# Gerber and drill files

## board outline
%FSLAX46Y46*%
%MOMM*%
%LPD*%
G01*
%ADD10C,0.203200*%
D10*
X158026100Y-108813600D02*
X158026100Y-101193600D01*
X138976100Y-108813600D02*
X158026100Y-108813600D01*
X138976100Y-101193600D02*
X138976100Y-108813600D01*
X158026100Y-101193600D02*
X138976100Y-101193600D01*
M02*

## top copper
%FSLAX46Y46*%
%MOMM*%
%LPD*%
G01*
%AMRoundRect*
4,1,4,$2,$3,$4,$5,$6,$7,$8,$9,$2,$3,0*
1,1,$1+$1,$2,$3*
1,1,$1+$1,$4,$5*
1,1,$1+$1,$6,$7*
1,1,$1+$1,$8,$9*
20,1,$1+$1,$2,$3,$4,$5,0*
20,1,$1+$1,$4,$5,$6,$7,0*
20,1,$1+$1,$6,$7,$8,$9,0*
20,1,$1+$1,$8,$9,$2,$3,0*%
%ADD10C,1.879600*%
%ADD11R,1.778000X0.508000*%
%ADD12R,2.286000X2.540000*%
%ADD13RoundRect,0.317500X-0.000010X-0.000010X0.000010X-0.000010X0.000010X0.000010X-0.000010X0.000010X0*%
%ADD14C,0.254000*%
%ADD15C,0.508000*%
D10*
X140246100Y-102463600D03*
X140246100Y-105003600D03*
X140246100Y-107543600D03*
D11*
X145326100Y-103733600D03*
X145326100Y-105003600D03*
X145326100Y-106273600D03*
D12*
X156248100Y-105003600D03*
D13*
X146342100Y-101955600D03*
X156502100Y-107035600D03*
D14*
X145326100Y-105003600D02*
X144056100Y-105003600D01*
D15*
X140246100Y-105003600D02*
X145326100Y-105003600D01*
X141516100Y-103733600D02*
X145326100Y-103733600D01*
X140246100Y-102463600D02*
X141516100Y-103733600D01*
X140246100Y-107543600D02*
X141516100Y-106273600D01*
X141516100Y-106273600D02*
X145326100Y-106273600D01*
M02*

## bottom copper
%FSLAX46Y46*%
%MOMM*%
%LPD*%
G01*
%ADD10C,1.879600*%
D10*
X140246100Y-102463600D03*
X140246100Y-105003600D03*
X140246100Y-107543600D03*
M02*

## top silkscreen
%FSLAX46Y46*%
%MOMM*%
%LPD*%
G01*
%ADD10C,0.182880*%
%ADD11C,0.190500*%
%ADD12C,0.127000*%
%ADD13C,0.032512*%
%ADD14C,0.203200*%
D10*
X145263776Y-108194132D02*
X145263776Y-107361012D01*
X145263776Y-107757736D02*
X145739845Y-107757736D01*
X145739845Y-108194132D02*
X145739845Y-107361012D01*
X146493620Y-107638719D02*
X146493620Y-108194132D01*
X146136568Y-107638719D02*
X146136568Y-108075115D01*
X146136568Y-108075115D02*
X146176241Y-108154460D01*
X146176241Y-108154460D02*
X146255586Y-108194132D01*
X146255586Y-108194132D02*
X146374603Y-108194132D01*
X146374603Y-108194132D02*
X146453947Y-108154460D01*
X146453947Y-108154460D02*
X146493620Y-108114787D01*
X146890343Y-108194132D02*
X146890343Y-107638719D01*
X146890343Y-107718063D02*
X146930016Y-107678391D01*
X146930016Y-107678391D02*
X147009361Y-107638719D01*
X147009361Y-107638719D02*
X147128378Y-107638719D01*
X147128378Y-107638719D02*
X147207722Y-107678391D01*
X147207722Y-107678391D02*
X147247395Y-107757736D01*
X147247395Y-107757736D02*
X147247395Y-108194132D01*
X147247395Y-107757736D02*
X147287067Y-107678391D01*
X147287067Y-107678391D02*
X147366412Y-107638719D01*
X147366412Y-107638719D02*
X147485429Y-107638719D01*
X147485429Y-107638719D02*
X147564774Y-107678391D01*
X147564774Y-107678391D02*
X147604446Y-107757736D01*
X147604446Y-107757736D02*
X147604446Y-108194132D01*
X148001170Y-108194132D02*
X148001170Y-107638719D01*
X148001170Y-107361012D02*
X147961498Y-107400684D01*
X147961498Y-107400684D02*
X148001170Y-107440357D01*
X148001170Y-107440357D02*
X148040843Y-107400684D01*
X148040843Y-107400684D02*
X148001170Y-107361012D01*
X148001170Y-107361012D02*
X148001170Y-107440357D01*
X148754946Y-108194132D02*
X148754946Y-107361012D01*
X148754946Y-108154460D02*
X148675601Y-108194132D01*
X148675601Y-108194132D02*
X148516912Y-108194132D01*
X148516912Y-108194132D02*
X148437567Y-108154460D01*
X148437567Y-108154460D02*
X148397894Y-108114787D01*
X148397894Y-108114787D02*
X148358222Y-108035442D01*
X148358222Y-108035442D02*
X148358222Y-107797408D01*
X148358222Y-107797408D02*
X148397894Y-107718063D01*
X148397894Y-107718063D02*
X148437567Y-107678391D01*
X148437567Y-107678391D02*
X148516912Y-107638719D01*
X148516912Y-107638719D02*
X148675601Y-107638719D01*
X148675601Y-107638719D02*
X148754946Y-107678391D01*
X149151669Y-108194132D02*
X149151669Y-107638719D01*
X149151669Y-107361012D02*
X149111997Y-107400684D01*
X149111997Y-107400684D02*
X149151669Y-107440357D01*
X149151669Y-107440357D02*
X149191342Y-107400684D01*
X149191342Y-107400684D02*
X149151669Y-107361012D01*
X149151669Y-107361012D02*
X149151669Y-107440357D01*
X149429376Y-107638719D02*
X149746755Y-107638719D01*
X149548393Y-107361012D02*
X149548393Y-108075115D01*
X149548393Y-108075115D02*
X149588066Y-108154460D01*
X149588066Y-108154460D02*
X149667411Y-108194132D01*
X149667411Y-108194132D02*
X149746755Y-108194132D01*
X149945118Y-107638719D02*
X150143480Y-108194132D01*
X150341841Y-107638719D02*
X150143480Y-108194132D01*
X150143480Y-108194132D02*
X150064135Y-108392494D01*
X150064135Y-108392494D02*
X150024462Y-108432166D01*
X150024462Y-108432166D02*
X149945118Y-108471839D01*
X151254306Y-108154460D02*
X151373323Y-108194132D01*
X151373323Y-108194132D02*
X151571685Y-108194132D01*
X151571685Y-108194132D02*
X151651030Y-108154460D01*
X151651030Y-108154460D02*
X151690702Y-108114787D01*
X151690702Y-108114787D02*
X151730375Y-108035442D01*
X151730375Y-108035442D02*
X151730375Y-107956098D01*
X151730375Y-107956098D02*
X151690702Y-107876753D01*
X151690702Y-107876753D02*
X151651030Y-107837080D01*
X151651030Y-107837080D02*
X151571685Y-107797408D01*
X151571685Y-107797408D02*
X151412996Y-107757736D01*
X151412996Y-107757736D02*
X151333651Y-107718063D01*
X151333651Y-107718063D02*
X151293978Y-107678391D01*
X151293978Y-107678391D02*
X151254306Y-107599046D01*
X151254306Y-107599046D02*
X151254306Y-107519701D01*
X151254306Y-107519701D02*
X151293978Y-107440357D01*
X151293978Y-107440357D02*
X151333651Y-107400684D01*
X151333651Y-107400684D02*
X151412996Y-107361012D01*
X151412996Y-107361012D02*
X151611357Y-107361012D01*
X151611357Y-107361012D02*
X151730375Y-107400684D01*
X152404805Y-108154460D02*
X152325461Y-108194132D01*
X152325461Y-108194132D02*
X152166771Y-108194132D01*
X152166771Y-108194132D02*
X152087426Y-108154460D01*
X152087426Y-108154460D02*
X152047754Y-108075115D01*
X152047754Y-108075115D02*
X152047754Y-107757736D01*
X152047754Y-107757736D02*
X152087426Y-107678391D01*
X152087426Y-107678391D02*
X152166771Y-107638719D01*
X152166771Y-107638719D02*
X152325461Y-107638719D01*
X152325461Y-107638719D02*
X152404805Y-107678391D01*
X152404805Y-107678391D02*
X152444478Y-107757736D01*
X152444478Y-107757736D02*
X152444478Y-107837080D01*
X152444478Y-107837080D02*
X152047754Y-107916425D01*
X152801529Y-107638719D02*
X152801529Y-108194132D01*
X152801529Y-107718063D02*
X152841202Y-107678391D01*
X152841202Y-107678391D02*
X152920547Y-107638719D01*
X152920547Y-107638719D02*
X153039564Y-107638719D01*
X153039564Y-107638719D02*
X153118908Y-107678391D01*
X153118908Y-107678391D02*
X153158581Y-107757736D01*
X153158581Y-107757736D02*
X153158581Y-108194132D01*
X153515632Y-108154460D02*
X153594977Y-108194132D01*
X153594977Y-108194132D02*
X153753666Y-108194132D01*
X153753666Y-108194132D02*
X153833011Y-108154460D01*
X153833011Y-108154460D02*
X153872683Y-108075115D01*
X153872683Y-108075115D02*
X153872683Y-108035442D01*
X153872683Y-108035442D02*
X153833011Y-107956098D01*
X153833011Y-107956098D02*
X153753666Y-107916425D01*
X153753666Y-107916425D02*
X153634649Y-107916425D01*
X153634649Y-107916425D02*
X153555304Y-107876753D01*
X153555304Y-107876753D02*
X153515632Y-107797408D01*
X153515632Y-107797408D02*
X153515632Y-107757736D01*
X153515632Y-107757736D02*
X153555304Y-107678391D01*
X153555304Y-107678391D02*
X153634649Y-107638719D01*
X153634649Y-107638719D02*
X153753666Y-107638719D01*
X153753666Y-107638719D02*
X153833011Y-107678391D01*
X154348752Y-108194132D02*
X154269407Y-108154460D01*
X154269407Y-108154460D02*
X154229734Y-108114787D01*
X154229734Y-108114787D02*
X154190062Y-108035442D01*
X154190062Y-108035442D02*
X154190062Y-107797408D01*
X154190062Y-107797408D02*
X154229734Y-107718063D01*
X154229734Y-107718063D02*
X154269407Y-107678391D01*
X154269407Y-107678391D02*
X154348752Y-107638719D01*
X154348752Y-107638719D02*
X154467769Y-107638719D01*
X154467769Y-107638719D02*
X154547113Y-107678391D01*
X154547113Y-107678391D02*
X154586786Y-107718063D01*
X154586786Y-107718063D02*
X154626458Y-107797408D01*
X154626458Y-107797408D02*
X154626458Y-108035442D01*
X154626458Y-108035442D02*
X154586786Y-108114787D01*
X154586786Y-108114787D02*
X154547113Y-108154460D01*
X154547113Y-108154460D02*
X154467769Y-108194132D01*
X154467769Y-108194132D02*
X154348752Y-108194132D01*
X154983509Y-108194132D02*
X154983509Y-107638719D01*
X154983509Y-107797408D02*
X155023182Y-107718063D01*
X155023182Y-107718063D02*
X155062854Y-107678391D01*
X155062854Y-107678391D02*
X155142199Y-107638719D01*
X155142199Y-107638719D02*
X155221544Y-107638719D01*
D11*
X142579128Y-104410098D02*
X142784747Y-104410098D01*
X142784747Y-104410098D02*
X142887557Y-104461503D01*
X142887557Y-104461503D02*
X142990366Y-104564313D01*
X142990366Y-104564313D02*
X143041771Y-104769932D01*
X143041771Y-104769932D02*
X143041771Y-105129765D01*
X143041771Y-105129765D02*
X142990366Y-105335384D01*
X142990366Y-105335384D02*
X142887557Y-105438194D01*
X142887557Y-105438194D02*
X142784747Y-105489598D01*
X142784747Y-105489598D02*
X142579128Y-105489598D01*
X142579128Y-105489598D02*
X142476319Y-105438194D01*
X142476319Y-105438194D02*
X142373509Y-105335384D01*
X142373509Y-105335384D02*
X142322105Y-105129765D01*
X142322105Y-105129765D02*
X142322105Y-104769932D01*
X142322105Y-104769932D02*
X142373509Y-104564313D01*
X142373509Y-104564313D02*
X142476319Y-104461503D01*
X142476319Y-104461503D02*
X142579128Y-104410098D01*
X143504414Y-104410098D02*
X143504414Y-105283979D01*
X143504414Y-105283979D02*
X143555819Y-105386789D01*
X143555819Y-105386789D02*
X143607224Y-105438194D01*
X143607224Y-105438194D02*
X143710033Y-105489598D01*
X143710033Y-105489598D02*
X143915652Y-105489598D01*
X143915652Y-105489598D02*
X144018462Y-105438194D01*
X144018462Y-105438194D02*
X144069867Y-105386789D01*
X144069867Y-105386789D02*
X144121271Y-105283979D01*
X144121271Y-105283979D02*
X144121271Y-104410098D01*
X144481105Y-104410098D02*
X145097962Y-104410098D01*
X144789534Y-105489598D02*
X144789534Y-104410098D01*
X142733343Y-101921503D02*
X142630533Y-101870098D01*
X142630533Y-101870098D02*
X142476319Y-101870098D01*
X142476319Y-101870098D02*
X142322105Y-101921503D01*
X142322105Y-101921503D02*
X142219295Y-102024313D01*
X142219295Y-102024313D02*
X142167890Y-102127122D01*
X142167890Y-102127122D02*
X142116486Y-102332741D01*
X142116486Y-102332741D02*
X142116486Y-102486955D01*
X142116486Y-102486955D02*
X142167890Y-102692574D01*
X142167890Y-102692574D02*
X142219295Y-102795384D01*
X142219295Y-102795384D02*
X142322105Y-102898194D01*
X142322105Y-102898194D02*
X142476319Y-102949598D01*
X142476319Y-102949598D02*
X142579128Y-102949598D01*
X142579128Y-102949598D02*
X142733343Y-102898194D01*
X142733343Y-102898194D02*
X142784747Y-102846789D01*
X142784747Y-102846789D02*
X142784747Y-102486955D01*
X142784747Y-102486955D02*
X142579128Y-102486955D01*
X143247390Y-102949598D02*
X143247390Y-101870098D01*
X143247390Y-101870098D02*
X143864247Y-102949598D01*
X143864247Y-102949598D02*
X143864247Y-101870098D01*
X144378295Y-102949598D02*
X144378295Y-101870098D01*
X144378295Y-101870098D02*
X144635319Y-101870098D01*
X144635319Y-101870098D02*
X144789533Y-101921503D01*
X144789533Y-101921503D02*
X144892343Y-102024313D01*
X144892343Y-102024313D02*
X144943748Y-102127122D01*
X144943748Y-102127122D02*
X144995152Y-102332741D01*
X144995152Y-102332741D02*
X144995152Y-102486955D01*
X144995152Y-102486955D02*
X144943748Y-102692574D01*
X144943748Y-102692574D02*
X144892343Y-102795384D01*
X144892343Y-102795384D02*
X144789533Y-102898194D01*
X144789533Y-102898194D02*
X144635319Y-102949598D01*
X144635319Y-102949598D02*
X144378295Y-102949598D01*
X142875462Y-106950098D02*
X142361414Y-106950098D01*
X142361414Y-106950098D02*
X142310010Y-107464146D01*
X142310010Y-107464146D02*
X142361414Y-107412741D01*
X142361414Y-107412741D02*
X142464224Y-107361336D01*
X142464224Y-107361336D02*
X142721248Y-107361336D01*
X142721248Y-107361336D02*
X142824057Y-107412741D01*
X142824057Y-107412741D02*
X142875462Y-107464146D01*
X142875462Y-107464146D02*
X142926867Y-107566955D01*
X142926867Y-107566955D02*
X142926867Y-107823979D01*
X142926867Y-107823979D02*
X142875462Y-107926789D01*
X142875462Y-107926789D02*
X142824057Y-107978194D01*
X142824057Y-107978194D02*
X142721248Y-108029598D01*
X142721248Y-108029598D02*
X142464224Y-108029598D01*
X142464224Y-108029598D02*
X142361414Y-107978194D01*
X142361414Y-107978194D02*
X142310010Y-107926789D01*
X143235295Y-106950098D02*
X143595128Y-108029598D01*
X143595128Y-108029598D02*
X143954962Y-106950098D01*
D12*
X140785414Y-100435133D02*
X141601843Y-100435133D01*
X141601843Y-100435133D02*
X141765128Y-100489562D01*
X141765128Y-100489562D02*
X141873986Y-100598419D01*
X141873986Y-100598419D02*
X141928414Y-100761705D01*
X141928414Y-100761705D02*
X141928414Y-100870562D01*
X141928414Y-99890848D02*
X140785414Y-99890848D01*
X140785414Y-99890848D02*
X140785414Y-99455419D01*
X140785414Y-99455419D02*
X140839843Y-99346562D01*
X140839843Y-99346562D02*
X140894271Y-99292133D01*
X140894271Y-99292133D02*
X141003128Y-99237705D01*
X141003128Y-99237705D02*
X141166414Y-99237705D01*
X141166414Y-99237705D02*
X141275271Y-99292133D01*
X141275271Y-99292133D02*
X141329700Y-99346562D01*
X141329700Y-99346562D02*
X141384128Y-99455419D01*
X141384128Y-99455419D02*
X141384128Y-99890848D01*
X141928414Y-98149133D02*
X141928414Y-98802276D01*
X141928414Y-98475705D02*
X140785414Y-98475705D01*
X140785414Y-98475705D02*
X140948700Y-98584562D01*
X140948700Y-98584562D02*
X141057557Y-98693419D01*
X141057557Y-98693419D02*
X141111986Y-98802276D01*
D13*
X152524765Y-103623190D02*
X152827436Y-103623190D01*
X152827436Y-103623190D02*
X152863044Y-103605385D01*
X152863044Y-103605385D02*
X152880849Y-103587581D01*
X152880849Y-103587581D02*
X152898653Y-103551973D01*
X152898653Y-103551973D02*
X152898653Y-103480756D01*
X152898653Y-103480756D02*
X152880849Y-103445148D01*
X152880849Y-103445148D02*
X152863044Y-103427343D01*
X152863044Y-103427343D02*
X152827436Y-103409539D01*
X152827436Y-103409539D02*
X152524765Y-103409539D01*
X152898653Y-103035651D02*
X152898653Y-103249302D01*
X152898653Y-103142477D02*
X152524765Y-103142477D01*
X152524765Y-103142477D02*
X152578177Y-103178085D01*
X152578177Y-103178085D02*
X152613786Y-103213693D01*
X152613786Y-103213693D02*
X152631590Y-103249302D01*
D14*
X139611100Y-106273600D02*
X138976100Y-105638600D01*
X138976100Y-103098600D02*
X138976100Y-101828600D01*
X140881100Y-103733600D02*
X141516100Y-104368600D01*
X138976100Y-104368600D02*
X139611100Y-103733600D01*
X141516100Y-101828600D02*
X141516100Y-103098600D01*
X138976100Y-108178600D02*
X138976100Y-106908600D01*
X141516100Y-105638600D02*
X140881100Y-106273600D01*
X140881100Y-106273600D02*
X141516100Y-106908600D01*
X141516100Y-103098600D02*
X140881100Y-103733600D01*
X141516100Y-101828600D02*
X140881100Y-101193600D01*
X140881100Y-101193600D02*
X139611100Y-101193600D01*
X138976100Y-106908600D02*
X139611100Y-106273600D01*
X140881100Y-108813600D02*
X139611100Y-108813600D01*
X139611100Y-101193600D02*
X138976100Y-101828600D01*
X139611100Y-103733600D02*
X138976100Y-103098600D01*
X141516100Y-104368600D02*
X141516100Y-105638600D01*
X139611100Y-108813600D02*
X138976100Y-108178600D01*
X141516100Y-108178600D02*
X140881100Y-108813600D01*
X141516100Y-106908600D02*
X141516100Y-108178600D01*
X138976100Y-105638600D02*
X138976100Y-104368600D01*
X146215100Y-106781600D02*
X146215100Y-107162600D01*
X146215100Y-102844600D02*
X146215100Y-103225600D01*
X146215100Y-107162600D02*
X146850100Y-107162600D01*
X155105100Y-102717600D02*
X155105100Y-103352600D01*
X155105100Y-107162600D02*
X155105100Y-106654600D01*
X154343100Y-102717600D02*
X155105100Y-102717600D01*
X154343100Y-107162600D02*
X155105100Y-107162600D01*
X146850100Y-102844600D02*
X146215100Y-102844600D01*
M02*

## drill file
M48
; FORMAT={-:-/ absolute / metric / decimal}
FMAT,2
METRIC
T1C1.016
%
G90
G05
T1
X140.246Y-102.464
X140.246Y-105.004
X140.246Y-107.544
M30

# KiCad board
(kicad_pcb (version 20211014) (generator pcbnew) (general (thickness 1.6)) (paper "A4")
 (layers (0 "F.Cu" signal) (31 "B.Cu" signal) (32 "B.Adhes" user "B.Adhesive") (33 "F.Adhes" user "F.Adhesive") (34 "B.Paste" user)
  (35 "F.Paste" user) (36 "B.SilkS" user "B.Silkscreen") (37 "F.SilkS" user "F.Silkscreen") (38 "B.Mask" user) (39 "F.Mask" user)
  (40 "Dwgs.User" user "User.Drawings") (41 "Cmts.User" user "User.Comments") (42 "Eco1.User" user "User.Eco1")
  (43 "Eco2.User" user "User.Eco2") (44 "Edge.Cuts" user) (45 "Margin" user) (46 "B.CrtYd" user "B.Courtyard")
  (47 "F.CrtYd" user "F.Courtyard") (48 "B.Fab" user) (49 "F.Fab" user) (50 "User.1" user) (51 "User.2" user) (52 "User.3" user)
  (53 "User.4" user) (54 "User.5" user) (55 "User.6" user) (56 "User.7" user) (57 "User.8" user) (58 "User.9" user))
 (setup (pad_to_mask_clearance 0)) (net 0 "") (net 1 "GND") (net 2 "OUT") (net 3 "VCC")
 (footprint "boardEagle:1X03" (layer "F.Cu") (at 140.2461 102.4636 -90)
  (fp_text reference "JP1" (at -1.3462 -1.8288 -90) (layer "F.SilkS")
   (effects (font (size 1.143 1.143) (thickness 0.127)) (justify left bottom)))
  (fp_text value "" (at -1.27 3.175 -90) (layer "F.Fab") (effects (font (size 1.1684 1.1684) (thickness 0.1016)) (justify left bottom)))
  (fp_line (start 3.81 0.635) (end 3.175 1.27) (layer "F.SilkS") (width 0.2032))
  (fp_line (start 0.635 1.27) (end -0.635 1.27) (layer "F.SilkS") (width 0.2032))
  (fp_line (start 1.27 -0.635) (end 1.905 -1.27) (layer "F.SilkS") (width 0.2032))
  (fp_line (start 1.905 1.27) (end 1.27 0.635) (layer "F.SilkS") (width 0.2032))
  (fp_line (start -0.635 -1.27) (end 0.635 -1.27) (layer "F.SilkS") (width 0.2032))
  (fp_line (start 5.715 1.27) (end 4.445 1.27) (layer "F.SilkS") (width 0.2032))
  (fp_line (start 3.175 -1.27) (end 3.81 -0.635) (layer "F.SilkS") (width 0.2032))
  (fp_line (start 3.81 -0.635) (end 4.445 -1.27) (layer "F.SilkS") (width 0.2032))
  (fp_line (start 0.635 -1.27) (end 1.27 -0.635) (layer "F.SilkS") (width 0.2032))
  (fp_line (start -0.635 -1.27) (end -1.27 -0.635) (layer "F.SilkS") (width 0.2032))
  (fp_line (start -1.27 -0.635) (end -1.27 0.635) (layer "F.SilkS") (width 0.2032))
  (fp_line (start 4.445 1.27) (end 3.81 0.635) (layer "F.SilkS") (width 0.2032))
  (fp_line (start 6.35 -0.635) (end 6.35 0.635) (layer "F.SilkS") (width 0.2032))
  (fp_line (start -1.27 0.635) (end -0.635 1.27) (layer "F.SilkS") (width 0.2032))
  (fp_line (start 1.27 0.635) (end 0.635 1.27) (layer "F.SilkS") (width 0.2032))
  (fp_line (start 1.905 -1.27) (end 3.175 -1.27) (layer "F.SilkS") (width 0.2032))
  (fp_line (start 6.35 0.635) (end 5.715 1.27) (layer "F.SilkS") (width 0.2032))
  (fp_line (start 5.715 -1.27) (end 6.35 -0.635) (layer "F.SilkS") (width 0.2032))
  (fp_line (start 4.445 -1.27) (end 5.715 -1.27) (layer "F.SilkS") (width 0.2032))
  (fp_line (start 3.175 1.27) (end 1.905 1.27) (layer "F.SilkS") (width 0.2032))
  (pad "1" thru_hole circle (at 0 0) (size 1.8796 1.8796) (drill 1.016) (layers *.Cu *.Mask) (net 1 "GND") (solder_mask_margin 0.1016))
  (pad "2" thru_hole circle (at 2.54 0) (size 1.8796 1.8796) (drill 1.016) (layers *.Cu *.Mask) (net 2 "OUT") (solder_mask_margin 0.1016))
  (pad "3" thru_hole circle (at 5.08 0) (size 1.8796 1.8796) (drill 1.016) (layers *.Cu *.Mask) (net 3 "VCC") (solder_mask_margin 0.1016)))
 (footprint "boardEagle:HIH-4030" (layer "F.Cu") (at 150.4061 105.0036 -90)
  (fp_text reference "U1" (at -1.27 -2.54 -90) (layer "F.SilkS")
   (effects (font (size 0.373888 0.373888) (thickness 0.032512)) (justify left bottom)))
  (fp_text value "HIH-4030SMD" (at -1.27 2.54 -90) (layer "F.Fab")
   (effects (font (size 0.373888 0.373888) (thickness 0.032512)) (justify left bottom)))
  (fp_line (start 1.778 4.191) (end 2.159 4.191) (layer "F.SilkS") (width 0.2032))
  (fp_line (start -2.159 4.191) (end -1.778 4.191) (layer "F.SilkS") (width 0.2032))
  (fp_line (start 2.159 4.191) (end 2.159 3.556) (layer "F.SilkS") (width 0.2032))
  (fp_line (start -2.286 -4.699) (end -1.651 -4.699) (layer "F.SilkS") (width 0.2032))
  (fp_line (start 2.159 -4.699) (end 1.651 -4.699) (layer "F.SilkS") (width 0.2032))
  (fp_line (start -2.286 -3.937) (end -2.286 -4.699) (layer "F.SilkS") (width 0.2032))
  (fp_line (start 2.159 -3.937) (end 2.159 -4.699) (layer "F.SilkS") (width 0.2032))
  (fp_line (start -2.159 3.556) (end -2.159 4.191) (layer "F.SilkS") (width 0.2032))
  (pad "1" smd rect (at -1.27 5.08 270) (size 0.508 1.778) (layers "F.Cu" "F.Paste" "F.Mask") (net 1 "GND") (solder_mask_margin 0.1016))
  (pad "2" smd rect (at 0 5.08 270) (size 0.508 1.778) (layers "F.Cu" "F.Paste" "F.Mask") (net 2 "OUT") (solder_mask_margin 0.1016))
  (pad "3" smd rect (at 1.27 5.08 270) (size 0.508 1.778) (layers "F.Cu" "F.Paste" "F.Mask") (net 3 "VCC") (solder_mask_margin 0.1016))
  (pad "NC" smd rect (at 0 -5.842 270) (size 2.54 2.286) (layers "F.Cu" "F.Paste" "F.Mask") (solder_mask_margin 0.1016)))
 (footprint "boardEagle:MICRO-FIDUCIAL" (layer "F.Cu") (at 146.3421 101.9556)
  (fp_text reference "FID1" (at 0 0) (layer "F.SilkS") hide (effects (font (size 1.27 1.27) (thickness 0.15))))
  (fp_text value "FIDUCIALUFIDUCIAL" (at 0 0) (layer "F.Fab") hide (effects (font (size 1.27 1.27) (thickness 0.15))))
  (pad "1" smd roundrect (at 0 0) (size 0.635 0.635) (layers "F.Cu" "F.Mask") (roundrect_rratio 0.5) (solder_mask_margin 0.1016)))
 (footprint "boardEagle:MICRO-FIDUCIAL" (layer "F.Cu") (at 156.5021 107.0356)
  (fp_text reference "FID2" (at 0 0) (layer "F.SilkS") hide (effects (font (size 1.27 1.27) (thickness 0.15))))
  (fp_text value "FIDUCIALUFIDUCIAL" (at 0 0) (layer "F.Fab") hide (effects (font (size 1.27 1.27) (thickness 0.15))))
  (pad "1" smd roundrect (at 0 0) (size 0.635 0.635) (layers "F.Cu" "F.Mask") (roundrect_rratio 0.5) (solder_mask_margin 0.1016)))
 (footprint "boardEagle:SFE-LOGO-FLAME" (layer "B.Cu") (at 149.3901 105.7656 90)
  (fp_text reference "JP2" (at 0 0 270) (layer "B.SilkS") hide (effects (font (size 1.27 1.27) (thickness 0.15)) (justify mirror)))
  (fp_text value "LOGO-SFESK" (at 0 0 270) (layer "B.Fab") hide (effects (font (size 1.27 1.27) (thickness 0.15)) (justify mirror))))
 (gr_line (start 158.0261 108.8136) (end 158.0261 101.1936) (layer "Edge.Cuts") (width 0.2032))
 (gr_line (start 138.9761 108.8136) (end 158.0261 108.8136) (layer "Edge.Cuts") (width 0.2032))
 (gr_line (start 138.9761 101.1936) (end 138.9761 108.8136) (layer "Edge.Cuts") (width 0.2032))
 (gr_line (start 158.0261 101.1936) (end 138.9761 101.1936) (layer "Edge.Cuts") (width 0.2032))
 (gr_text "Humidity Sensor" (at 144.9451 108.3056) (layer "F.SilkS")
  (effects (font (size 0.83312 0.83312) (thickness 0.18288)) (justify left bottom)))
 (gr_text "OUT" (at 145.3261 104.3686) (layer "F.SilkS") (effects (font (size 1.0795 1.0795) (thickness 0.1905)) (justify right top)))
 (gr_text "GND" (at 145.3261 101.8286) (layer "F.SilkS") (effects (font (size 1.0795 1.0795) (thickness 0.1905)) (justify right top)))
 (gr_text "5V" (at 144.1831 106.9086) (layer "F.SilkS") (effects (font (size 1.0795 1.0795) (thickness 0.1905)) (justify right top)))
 (segment (start 145.3261 105.0036) (end 144.0561 105.0036) (width 0.254) (layer "F.Cu") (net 2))
 (segment (start 140.2461 105.0036) (end 145.3261 105.0036) (width 0.508) (layer "F.Cu") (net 2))
 (segment (start 141.5161 103.7336) (end 145.3261 103.7336) (width 0.508) (layer "F.Cu") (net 1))
 (segment (start 140.2461 102.4636) (end 141.5161 103.7336) (width 0.508) (layer "F.Cu") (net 1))
 (segment (start 140.2461 107.5436) (end 141.5161 106.2736) (width 0.508) (layer "F.Cu") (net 3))
 (segment (start 141.5161 106.2736) (end 145.3261 106.2736) (width 0.508) (layer "F.Cu") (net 3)))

